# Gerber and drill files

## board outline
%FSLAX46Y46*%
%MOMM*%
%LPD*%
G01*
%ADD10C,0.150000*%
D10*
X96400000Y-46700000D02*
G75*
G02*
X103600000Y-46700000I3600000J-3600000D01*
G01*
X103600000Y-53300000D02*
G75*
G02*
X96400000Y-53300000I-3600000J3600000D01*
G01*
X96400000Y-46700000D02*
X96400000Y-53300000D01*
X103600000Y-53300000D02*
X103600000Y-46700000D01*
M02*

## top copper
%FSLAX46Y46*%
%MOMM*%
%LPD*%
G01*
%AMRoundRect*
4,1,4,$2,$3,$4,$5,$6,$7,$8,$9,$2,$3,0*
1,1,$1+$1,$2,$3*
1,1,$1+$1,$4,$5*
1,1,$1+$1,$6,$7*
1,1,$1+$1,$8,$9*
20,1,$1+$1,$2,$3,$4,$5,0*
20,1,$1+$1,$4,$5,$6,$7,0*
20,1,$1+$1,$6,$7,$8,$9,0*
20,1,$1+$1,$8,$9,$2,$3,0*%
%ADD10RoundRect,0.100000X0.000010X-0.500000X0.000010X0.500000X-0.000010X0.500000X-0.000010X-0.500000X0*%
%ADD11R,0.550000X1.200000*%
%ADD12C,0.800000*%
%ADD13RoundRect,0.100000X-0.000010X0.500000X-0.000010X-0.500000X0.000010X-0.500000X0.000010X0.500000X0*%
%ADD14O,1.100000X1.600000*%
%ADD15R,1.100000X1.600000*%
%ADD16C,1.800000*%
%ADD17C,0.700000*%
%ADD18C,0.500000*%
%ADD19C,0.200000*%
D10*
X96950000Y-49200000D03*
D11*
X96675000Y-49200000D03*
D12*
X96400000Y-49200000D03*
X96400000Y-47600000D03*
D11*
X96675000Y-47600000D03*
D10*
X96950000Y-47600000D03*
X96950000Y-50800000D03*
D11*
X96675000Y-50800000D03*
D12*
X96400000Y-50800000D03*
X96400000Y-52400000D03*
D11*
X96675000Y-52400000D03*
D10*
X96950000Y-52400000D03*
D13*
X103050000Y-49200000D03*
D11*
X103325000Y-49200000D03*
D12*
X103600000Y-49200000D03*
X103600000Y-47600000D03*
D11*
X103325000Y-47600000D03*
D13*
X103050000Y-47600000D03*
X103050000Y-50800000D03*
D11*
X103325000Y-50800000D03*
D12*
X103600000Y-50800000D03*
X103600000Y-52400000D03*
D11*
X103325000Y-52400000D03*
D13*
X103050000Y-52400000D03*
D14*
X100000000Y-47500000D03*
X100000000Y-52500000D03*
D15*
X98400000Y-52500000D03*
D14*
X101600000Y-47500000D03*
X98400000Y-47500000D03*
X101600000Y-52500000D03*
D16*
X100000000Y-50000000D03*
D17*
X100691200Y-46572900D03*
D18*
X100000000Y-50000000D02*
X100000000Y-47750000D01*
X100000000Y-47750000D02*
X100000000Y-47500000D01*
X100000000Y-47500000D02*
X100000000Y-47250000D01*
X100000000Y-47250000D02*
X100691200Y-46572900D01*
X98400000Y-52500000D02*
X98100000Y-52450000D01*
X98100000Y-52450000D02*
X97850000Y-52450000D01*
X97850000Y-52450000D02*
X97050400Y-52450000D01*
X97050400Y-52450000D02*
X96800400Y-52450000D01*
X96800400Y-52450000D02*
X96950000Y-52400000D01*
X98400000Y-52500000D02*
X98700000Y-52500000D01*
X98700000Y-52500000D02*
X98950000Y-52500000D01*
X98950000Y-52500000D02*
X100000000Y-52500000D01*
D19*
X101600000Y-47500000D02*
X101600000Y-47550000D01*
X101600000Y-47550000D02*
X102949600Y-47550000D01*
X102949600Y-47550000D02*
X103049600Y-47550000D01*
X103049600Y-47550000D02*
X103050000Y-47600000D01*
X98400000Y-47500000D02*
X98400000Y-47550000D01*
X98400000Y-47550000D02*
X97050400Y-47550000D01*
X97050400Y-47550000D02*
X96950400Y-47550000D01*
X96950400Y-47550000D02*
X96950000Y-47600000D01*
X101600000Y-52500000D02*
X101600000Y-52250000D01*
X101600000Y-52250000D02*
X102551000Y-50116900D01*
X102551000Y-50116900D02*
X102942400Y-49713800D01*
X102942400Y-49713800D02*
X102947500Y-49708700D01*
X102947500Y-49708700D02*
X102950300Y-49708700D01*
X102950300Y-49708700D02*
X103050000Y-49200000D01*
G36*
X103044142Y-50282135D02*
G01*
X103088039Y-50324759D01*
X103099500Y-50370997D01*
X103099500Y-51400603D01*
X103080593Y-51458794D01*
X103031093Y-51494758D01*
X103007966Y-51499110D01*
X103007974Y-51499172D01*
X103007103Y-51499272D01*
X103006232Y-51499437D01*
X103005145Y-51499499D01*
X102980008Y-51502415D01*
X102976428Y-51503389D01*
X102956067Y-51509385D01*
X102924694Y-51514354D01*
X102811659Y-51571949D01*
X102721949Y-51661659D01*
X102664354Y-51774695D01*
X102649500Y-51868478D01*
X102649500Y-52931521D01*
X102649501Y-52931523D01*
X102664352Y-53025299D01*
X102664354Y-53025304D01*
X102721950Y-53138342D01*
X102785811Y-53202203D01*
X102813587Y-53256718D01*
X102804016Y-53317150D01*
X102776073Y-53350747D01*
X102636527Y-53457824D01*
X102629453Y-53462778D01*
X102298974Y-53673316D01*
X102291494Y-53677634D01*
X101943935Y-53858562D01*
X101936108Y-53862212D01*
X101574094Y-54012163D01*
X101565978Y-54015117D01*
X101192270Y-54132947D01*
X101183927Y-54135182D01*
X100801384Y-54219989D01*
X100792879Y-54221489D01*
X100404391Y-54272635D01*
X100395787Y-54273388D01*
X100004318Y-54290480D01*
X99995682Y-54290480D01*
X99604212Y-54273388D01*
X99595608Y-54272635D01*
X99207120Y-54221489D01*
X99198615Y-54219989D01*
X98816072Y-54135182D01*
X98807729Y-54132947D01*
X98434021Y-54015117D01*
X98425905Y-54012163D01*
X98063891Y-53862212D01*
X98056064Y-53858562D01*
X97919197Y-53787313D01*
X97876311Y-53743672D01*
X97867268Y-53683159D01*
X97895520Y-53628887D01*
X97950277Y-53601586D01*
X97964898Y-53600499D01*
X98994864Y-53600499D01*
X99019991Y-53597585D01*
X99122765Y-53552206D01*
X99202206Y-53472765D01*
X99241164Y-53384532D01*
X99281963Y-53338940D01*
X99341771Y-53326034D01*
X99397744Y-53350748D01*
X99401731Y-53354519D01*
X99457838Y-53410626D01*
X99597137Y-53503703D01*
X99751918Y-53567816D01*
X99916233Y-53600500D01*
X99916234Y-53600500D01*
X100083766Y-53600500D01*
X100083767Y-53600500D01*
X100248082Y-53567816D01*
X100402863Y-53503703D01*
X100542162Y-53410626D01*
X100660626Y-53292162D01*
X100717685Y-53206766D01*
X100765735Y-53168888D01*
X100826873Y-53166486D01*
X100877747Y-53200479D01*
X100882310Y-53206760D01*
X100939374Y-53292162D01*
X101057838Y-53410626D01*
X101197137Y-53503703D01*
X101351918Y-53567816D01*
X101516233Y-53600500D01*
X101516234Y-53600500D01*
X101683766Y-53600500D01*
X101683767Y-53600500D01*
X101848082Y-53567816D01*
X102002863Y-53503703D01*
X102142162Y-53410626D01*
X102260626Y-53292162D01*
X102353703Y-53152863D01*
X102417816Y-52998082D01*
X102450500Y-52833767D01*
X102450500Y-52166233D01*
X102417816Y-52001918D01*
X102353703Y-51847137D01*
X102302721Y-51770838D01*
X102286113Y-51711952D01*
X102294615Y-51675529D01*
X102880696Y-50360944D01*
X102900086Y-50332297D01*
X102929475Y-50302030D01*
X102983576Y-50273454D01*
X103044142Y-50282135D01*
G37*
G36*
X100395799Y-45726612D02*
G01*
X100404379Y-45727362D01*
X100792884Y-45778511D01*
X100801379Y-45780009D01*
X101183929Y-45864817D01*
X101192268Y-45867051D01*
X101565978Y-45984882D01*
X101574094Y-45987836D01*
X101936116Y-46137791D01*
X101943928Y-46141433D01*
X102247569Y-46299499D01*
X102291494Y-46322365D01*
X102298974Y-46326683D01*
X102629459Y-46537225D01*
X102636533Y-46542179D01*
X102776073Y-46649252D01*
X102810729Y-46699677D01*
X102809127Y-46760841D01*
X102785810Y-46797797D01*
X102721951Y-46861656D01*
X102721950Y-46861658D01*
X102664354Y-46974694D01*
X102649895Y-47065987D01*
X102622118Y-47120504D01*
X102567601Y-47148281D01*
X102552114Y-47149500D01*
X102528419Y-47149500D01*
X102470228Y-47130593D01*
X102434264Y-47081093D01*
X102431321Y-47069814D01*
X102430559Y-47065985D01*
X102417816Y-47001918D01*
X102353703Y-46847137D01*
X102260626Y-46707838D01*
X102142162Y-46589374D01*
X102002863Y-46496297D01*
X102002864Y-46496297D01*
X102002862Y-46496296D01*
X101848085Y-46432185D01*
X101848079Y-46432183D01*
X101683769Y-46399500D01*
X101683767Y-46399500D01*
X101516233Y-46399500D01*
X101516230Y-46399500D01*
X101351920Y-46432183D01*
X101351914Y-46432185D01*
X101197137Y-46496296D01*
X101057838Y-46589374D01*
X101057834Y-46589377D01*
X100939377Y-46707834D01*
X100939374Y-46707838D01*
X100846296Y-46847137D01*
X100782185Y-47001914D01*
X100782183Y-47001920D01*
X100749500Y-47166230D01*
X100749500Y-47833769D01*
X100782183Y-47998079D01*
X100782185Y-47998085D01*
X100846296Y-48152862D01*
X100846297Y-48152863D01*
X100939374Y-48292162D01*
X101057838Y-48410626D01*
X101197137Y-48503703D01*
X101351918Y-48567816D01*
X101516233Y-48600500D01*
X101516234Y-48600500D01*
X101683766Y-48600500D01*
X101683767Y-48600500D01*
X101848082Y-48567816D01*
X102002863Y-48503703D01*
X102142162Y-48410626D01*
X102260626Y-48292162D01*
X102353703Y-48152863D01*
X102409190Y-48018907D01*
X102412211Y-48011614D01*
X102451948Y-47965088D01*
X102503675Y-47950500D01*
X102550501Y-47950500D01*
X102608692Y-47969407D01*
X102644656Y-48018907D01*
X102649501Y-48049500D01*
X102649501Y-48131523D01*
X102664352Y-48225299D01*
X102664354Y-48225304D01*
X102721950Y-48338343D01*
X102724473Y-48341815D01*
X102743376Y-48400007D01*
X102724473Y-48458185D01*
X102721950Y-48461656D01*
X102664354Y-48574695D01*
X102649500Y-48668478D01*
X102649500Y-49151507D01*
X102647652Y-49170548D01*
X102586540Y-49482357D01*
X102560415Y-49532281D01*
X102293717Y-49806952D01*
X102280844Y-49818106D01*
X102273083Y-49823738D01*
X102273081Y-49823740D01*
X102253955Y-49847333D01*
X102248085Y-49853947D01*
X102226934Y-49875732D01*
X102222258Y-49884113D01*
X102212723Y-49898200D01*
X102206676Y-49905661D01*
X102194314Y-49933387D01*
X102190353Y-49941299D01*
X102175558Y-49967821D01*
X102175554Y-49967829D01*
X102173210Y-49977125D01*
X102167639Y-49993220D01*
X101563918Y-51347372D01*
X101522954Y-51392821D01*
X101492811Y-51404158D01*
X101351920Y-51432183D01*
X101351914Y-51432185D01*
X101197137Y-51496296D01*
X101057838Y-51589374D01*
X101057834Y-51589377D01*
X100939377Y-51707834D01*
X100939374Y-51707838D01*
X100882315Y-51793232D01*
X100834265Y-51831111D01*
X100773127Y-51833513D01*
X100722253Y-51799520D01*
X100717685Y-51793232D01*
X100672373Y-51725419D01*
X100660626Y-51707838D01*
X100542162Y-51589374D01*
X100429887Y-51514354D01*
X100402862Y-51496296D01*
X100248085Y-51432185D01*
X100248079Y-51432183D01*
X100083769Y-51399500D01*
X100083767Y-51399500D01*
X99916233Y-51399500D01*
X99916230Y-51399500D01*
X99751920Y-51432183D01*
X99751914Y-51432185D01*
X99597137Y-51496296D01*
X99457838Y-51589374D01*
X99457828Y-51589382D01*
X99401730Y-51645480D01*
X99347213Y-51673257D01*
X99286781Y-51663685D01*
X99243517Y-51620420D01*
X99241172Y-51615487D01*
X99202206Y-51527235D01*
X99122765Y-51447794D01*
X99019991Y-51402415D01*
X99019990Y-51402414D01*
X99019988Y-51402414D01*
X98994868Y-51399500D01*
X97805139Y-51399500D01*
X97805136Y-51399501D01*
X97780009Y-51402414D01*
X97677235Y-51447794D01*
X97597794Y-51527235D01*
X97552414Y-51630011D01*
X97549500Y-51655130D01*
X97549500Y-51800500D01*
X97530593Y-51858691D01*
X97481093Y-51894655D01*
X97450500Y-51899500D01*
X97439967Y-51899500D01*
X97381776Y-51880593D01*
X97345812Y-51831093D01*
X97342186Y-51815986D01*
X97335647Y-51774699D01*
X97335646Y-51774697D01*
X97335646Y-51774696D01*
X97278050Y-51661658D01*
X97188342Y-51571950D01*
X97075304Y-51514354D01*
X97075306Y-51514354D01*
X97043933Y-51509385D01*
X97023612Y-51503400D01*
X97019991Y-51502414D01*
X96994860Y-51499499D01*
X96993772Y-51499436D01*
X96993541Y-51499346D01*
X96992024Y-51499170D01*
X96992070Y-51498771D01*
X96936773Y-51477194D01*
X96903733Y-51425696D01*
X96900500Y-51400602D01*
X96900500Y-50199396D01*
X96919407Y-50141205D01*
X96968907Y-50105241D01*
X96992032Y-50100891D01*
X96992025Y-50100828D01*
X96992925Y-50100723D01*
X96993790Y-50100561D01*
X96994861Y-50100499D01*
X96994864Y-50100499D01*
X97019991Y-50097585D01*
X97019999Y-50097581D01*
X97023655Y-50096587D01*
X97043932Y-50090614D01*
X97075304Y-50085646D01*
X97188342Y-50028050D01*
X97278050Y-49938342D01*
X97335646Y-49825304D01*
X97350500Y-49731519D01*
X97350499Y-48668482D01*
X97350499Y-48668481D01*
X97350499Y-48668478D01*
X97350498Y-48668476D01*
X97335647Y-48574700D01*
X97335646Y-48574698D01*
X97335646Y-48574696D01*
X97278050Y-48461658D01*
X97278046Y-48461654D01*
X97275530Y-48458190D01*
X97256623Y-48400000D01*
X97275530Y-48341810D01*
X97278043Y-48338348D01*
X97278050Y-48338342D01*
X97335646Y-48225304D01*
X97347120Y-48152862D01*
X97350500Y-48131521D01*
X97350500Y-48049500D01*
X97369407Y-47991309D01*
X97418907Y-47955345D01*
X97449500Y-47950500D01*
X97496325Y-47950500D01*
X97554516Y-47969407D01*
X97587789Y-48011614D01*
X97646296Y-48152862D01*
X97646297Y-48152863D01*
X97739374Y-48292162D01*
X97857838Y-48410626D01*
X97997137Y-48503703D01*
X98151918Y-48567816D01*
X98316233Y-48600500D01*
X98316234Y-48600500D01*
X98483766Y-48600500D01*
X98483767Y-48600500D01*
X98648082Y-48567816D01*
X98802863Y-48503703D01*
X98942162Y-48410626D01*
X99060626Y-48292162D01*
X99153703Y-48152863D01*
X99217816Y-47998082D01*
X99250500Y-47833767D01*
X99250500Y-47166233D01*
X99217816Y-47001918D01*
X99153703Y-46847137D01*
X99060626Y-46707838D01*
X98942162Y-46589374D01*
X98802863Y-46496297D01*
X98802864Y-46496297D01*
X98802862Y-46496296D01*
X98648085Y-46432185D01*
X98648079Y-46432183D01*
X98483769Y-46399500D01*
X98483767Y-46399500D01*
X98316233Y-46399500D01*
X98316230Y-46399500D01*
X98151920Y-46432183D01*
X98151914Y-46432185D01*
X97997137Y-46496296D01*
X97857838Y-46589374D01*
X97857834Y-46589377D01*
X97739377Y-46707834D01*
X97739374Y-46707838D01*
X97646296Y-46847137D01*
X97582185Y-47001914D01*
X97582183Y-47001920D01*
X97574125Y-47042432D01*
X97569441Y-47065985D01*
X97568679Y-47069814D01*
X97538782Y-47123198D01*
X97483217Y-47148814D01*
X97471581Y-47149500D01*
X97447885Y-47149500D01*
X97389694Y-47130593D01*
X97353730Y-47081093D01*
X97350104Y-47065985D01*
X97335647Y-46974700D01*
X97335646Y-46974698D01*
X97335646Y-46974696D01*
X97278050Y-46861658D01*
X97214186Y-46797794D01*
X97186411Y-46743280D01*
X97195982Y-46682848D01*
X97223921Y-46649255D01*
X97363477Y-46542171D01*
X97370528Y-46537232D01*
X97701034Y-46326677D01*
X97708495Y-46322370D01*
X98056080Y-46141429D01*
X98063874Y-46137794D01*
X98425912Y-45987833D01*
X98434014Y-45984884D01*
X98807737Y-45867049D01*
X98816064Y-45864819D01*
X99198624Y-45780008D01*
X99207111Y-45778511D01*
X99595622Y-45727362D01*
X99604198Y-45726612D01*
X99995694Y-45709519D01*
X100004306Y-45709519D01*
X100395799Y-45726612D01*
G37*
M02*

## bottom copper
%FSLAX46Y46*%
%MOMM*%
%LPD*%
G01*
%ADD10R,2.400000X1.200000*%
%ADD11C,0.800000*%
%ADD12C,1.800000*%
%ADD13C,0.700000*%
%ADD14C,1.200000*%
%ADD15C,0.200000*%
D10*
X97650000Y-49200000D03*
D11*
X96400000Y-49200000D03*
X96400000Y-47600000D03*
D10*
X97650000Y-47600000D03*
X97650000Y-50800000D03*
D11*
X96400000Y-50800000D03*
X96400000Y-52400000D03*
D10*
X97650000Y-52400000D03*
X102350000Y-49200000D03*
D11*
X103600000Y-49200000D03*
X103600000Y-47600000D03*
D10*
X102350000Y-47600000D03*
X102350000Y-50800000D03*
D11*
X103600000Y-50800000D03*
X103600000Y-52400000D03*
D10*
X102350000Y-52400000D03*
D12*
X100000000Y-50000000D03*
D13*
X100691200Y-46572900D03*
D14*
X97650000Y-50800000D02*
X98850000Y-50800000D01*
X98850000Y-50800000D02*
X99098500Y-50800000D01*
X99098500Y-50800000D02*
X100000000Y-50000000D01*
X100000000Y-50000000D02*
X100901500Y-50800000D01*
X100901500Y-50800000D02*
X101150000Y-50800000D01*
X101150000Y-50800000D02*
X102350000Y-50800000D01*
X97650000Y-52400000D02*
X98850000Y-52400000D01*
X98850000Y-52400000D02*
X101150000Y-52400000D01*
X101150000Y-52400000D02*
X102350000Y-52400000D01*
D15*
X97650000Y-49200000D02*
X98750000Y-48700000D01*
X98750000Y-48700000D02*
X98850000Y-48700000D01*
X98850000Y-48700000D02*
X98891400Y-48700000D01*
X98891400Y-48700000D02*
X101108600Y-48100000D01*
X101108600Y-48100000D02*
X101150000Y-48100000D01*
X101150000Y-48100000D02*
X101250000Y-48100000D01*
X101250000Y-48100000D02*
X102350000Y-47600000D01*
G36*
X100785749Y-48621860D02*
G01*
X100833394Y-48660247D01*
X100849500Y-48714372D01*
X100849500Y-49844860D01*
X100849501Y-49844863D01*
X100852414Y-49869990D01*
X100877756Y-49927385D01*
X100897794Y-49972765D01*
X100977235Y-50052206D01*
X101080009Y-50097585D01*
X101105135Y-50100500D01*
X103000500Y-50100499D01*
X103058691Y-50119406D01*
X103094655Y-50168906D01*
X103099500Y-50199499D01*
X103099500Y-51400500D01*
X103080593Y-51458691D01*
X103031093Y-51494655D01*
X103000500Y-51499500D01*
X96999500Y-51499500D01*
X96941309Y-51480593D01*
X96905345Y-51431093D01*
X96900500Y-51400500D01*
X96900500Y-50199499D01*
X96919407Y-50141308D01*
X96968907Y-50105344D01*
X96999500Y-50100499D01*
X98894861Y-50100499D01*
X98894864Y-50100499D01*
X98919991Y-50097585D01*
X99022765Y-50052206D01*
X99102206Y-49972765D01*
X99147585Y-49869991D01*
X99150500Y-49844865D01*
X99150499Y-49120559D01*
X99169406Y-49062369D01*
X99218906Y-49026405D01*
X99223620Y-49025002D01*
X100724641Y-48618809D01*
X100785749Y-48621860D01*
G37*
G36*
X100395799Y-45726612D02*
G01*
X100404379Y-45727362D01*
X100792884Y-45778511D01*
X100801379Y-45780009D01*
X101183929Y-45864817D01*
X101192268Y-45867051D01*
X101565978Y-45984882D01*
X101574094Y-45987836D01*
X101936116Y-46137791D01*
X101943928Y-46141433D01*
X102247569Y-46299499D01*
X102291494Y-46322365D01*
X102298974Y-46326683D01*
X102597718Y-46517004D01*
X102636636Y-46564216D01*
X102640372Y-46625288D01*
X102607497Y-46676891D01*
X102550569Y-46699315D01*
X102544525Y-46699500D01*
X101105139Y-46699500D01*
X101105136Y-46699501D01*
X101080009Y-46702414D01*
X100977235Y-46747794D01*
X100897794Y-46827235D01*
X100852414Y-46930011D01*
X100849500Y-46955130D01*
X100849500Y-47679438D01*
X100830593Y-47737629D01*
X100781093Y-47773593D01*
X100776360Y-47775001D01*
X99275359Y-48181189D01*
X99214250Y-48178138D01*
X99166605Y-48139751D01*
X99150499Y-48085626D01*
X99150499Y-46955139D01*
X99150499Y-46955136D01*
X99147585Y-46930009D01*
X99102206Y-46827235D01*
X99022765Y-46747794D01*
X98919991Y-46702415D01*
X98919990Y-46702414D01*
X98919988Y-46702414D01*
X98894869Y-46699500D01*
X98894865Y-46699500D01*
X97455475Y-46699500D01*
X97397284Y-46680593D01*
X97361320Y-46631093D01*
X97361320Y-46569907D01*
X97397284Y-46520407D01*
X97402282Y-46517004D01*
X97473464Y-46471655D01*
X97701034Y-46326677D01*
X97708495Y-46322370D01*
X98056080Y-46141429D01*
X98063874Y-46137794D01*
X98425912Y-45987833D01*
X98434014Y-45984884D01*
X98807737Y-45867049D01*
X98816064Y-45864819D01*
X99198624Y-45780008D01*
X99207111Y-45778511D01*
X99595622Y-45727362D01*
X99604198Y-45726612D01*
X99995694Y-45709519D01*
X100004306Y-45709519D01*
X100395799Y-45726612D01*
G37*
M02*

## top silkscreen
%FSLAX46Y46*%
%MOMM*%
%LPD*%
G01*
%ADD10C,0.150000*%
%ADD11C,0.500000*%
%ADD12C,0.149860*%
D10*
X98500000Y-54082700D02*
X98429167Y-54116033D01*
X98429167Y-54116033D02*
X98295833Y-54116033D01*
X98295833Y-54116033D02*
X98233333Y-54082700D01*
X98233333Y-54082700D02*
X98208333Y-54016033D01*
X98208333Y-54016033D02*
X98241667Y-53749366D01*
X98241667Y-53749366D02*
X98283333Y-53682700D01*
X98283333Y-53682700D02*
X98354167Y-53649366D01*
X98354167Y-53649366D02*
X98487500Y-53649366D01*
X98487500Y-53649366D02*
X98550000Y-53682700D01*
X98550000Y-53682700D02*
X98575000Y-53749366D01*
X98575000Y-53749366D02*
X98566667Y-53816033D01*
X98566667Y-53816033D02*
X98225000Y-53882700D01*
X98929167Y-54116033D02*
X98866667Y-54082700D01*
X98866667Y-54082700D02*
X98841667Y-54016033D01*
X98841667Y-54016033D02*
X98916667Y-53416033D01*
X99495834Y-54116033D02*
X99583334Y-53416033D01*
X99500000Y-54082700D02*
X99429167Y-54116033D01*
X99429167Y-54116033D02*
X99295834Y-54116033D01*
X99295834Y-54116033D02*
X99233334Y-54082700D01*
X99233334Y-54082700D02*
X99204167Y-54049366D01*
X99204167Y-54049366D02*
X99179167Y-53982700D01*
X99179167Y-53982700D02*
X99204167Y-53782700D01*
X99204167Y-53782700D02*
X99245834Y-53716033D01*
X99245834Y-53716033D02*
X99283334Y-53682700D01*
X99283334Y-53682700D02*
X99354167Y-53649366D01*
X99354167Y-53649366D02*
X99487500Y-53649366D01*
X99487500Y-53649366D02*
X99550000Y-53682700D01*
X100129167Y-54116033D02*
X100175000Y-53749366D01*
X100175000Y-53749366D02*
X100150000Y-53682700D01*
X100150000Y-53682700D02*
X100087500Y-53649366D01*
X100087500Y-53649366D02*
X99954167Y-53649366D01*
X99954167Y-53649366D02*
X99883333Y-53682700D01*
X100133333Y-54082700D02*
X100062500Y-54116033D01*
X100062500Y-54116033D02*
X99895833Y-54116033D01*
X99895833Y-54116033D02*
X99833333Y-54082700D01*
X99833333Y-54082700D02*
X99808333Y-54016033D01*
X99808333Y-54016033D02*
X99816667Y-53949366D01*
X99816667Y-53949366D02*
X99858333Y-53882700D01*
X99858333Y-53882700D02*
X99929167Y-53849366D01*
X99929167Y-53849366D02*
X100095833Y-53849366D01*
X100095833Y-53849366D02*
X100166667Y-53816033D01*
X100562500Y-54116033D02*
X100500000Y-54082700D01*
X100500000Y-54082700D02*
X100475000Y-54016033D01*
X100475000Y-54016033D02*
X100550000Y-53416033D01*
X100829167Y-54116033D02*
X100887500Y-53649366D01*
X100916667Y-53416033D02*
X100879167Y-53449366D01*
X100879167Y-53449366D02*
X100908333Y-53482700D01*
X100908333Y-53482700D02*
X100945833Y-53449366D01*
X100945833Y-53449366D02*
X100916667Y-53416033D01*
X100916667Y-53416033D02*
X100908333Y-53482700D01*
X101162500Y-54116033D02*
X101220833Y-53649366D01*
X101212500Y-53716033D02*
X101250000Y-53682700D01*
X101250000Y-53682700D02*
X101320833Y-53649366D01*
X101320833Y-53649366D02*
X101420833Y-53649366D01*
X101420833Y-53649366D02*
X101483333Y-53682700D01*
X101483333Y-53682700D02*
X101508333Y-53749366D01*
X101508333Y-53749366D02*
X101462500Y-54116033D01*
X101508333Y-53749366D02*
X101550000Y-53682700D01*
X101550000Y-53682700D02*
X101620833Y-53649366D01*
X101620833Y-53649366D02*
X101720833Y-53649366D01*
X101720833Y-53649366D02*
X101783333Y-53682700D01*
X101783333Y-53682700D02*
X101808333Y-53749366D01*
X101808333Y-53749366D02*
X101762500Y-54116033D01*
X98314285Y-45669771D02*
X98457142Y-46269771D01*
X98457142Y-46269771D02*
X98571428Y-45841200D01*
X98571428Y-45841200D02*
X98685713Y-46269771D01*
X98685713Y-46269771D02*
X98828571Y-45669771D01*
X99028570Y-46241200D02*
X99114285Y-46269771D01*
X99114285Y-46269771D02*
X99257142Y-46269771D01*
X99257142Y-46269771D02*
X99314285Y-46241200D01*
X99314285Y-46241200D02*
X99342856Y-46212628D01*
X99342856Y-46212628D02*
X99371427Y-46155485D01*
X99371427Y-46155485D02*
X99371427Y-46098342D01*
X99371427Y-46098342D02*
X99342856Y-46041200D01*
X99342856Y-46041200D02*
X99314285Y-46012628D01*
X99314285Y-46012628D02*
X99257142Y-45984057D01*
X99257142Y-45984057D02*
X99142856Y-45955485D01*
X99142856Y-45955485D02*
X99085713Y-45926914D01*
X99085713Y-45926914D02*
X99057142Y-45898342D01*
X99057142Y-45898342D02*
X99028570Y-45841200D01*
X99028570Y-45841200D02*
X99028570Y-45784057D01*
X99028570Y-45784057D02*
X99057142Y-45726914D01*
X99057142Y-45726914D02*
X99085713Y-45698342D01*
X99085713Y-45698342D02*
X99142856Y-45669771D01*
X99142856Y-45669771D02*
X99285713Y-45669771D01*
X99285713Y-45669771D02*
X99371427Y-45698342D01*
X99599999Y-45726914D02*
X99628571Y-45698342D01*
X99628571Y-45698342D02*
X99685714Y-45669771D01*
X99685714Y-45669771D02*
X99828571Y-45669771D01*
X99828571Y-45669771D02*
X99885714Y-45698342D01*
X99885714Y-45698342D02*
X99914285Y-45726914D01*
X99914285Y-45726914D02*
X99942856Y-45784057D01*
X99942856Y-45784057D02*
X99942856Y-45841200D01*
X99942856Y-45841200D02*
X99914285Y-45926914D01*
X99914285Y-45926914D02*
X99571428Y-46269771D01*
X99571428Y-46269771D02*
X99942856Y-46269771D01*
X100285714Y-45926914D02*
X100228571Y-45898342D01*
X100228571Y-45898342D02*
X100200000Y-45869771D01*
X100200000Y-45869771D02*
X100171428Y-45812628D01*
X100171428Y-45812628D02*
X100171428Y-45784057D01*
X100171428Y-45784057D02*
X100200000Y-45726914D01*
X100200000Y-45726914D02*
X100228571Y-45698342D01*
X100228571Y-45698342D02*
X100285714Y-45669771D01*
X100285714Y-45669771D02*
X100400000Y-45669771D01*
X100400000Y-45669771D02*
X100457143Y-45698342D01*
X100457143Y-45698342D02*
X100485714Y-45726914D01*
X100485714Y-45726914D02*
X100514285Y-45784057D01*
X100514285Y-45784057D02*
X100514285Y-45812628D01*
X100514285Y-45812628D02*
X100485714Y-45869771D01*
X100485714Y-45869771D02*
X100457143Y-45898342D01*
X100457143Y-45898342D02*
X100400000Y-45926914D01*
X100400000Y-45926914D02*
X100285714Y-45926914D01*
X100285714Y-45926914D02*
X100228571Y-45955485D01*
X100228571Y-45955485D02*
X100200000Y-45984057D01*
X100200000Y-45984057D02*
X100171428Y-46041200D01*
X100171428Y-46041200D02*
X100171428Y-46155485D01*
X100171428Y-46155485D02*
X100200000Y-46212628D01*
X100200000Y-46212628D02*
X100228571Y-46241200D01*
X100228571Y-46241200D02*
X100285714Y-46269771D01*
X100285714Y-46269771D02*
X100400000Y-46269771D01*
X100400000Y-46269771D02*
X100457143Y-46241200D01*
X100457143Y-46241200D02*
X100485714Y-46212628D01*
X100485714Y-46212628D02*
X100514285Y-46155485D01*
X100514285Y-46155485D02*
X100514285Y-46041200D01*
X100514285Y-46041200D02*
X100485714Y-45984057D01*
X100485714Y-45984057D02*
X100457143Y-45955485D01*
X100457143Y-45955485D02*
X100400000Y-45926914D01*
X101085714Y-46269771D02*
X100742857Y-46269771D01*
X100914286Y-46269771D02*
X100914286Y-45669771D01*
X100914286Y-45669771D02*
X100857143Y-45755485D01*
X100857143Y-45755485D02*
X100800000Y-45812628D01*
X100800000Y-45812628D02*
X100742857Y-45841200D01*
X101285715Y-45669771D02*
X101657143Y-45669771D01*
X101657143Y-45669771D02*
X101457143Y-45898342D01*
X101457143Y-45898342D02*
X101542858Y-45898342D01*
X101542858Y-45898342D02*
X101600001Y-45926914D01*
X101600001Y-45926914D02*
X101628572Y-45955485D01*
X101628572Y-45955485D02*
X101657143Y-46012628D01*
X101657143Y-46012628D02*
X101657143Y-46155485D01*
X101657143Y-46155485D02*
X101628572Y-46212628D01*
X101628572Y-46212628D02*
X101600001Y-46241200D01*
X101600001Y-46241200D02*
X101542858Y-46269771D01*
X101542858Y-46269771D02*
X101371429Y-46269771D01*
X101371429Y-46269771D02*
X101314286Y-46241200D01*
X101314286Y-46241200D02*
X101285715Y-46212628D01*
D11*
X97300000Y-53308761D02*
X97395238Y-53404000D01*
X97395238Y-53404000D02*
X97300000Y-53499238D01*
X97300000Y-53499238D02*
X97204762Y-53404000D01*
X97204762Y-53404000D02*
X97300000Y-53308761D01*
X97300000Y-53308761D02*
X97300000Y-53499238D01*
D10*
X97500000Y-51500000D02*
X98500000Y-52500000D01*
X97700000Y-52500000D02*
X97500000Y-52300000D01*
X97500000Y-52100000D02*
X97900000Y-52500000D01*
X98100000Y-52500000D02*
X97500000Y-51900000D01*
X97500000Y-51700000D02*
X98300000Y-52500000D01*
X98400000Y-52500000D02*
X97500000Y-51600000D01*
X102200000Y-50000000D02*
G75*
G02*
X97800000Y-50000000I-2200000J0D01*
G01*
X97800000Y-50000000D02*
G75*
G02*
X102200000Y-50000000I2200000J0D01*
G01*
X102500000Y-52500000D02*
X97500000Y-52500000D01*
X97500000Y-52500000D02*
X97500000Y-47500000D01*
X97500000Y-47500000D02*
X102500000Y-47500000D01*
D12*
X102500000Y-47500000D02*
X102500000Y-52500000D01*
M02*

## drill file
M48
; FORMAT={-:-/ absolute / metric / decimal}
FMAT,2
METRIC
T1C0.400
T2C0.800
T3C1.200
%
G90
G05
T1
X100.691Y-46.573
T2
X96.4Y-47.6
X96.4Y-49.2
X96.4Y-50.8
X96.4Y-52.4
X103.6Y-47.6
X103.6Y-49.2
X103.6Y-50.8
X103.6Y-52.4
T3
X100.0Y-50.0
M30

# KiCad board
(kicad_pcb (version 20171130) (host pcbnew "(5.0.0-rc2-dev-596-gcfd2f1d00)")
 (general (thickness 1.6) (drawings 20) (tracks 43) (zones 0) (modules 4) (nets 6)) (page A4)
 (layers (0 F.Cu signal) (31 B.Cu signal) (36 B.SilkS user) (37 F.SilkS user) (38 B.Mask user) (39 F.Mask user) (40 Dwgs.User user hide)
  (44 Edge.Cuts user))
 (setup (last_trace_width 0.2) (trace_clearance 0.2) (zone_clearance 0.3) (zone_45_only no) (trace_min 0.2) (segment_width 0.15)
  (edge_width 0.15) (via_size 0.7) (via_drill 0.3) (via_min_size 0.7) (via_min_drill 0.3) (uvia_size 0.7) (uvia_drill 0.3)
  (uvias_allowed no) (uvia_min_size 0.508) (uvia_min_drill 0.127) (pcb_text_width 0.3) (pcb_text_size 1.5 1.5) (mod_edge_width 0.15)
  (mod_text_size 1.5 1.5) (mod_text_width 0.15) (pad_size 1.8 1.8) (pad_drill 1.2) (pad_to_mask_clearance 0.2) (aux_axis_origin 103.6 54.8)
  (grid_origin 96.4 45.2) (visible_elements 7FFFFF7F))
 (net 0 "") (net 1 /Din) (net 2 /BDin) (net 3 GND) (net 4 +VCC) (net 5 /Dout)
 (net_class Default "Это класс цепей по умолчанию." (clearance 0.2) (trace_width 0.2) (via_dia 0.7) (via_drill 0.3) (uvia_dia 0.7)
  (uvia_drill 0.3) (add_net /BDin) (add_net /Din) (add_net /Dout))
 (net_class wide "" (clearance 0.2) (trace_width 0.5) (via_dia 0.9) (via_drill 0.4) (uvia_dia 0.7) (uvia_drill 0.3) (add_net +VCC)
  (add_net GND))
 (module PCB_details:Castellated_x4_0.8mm (layer F.Cu) (at 96.4 52.4 90)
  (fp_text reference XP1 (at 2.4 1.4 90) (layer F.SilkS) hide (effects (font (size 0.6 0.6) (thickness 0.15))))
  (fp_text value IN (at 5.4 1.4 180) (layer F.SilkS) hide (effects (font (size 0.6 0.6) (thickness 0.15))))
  (pad 3 smd roundrect (at 3.2 0.55 90) (size 1.2 0.2) (layers F.Cu F.Mask) (roundrect_rratio 0.5) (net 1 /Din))
  (pad 3 smd rect (at 3.2 1.25 90) (size 1.2 2.4) (layers B.Cu B.Mask) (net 1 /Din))
  (pad 3 smd rect (at 3.2 0.275 90) (size 1.2 0.55) (layers F.Cu F.Mask) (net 1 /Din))
  (pad 3 thru_hole circle (at 3.2 0 90) (size 0.8 0.8) (drill 0.8) (layers *.Cu) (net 1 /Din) (clearance 0.001))
  (pad 4 thru_hole circle (at 4.8 0 90) (size 0.8 0.8) (drill 0.8) (layers *.Cu) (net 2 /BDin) (clearance 0.001))
  (pad 4 smd rect (at 4.8 0.275 90) (size 1.2 0.55) (layers F.Cu F.Mask) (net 2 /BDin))
  (pad 4 smd rect (at 4.8 1.25 90) (size 1.2 2.4) (layers B.Cu B.Mask) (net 2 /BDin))
  (pad 4 smd roundrect (at 4.8 0.55 90) (size 1.2 0.2) (layers F.Cu F.Mask) (roundrect_rratio 0.5) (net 2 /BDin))
  (pad 2 smd roundrect (at 1.6 0.55 90) (size 1.2 0.2) (layers F.Cu F.Mask) (roundrect_rratio 0.5) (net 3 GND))
  (pad 2 smd rect (at 1.6 1.25 90) (size 1.2 2.4) (layers B.Cu B.Mask) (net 3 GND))
  (pad 2 smd rect (at 1.6 0.275 90) (size 1.2 0.55) (layers F.Cu F.Mask) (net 3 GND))
  (pad 2 thru_hole circle (at 1.6 0 90) (size 0.8 0.8) (drill 0.8) (layers *.Cu) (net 3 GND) (clearance 0.001))
  (pad 1 thru_hole circle (at 0 0 90) (size 0.8 0.8) (drill 0.8) (layers *.Cu) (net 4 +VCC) (clearance 0.001))
  (pad 1 smd rect (at 0 0.275 90) (size 1.2 0.55) (layers F.Cu F.Mask) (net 4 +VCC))
  (pad 1 smd rect (at 0 1.25 90) (size 1.2 2.4) (layers B.Cu B.Mask) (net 4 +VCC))
  (pad 1 smd roundrect (at 0 0.55 90) (size 1.2 0.2) (layers F.Cu F.Mask) (roundrect_rratio 0.5) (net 4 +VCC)))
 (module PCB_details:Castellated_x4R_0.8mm (layer F.Cu) (at 103.6 52.4 270)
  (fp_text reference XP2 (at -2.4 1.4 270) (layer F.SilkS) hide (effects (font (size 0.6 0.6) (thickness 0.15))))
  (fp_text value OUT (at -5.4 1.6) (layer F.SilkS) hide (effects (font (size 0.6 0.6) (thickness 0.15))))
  (pad 3 smd roundrect (at -3.2 0.55 270) (size 1.2 0.2) (layers F.Cu F.Mask) (roundrect_rratio 0.5) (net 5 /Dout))
  (pad 3 smd rect (at -3.2 1.25 270) (size 1.2 2.4) (layers B.Cu B.Mask) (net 5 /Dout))
  (pad 3 smd rect (at -3.2 0.275 270) (size 1.2 0.55) (layers F.Cu F.Mask) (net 5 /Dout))
  (pad 3 thru_hole circle (at -3.2 0 270) (size 0.8 0.8) (drill 0.8) (layers *.Cu) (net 5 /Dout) (clearance 0.001))
  (pad 4 thru_hole circle (at -4.8 0 270) (size 0.8 0.8) (drill 0.8) (layers *.Cu) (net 1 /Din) (clearance 0.001))
  (pad 4 smd rect (at -4.8 0.275 270) (size 1.2 0.55) (layers F.Cu F.Mask) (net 1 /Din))
  (pad 4 smd rect (at -4.8 1.25 270) (size 1.2 2.4) (layers B.Cu B.Mask) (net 1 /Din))
  (pad 4 smd roundrect (at -4.8 0.55 270) (size 1.2 0.2) (layers F.Cu F.Mask) (roundrect_rratio 0.5) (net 1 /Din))
  (pad 2 smd roundrect (at -1.6 0.55 270) (size 1.2 0.2) (layers F.Cu F.Mask) (roundrect_rratio 0.5) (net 3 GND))
  (pad 2 smd rect (at -1.6 1.25 270) (size 1.2 2.4) (layers B.Cu B.Mask) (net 3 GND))
  (pad 2 smd rect (at -1.6 0.275 270) (size 1.2 0.55) (layers F.Cu F.Mask) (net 3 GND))
  (pad 2 thru_hole circle (at -1.6 0 270) (size 0.8 0.8) (drill 0.8) (layers *.Cu) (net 3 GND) (clearance 0.001))
  (pad 1 thru_hole circle (at 0 0 270) (size 0.8 0.8) (drill 0.8) (layers *.Cu) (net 4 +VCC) (clearance 0.001))
  (pad 1 smd rect (at 0 0.275 270) (size 1.2 0.55) (layers F.Cu F.Mask) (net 4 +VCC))
  (pad 1 smd rect (at 0 1.25 270) (size 1.2 2.4) (layers B.Cu B.Mask) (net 4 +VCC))
  (pad 1 smd roundrect (at 0 0.55 270) (size 1.2 0.2) (layers F.Cu F.Mask) (roundrect_rratio 0.5) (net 4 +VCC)))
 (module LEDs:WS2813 (layer F.Cu) (at 100 50 270)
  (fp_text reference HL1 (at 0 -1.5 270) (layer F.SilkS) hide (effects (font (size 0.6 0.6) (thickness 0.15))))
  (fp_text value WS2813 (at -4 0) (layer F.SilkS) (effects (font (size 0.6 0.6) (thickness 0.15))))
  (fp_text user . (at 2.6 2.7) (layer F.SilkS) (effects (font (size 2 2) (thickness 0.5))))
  (fp_line (start 1.5 2.5) (end 2.5 1.5) (layer F.SilkS) (width 0.15))
  (fp_line (start 2.5 2.3) (end 2.3 2.5) (layer F.SilkS) (width 0.15))
  (fp_line (start 2.1 2.5) (end 2.5 2.1) (layer F.SilkS) (width 0.15))
  (fp_line (start 2.5 1.9) (end 1.9 2.5) (layer F.SilkS) (width 0.15))
  (fp_line (start 1.7 2.5) (end 2.5 1.7) (layer F.SilkS) (width 0.15))
  (fp_line (start 2.5 1.6) (end 1.6 2.5) (layer F.SilkS) (width 0.15))
  (fp_circle (center 0 0) (end 0 2.2) (layer F.SilkS) (width 0.15))
  (fp_line (start 2.5 -2.5) (end 2.5 2.5) (layer F.SilkS) (width 0.15))
  (fp_line (start 2.5 2.5) (end -2.5 2.5) (layer F.SilkS) (width 0.15))
  (fp_line (start -2.5 2.5) (end -2.5 -2.5) (layer F.SilkS) (width 0.15))
  (fp_line (start -2.5 -2.5) (end 2.5 -2.5) (layer F.SilkS) (width 0.14986))
  (pad 5 smd oval (at -2.5 0 270) (size 1.6 1.1) (layers F.Cu F.Mask) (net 3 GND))
  (pad 2 smd oval (at 2.5 0 270) (size 1.6 1.1) (layers F.Cu F.Mask) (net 4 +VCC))
  (pad 1 smd rect (at 2.5 1.6 270) (size 1.6 1.1) (layers F.Cu F.Mask) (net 4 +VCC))
  (pad 4 smd oval (at -2.5 -1.6 270) (size 1.6 1.1) (layers F.Cu F.Mask) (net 1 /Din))
  (pad 6 smd oval (at -2.5 1.6 270) (size 1.6 1.1) (layers F.Cu F.Mask) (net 2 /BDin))
  (pad 3 smd oval (at 2.5 -1.6 270) (size 1.6 1.1) (layers F.Cu F.Mask) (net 5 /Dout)))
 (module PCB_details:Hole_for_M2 (layer F.Cu) (at 100 50 270)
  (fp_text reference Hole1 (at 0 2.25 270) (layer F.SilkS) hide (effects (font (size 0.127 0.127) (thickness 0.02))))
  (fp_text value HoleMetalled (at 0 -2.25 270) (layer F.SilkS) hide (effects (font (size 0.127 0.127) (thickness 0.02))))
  (pad H thru_hole circle (at 0 0 270) (size 1.8 1.8) (drill 1.2) (layers *.Cu *.Mask) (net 3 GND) (zone_connect 2)))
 (gr_arc (start 100 50.3) (end 96.4 46.7) (angle 90) (layer Edge.Cuts) (width 0.15))
 (gr_arc (start 100 49.7) (end 103.6 53.3) (angle 90) (layer Edge.Cuts) (width 0.15))
 (gr_line (start 96.4 46.7) (end 96.4 53.3) (angle 90) (layer Edge.Cuts) (width 0.15))
 (gr_line (start 103.6 53.3) (end 103.6 46.7) (angle 90) (layer Edge.Cuts) (width 0.15))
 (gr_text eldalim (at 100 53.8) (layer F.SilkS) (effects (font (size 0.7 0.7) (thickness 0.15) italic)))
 (segment (start 100 50) (end 100 47.75) (width 0.5) (layer F.Cu) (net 3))
 (segment (start 100 47.75) (end 100 47.5) (width 0.5) (layer F.Cu) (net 3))
 (segment (start 100 47.5) (end 100 47.25) (width 0.5) (layer F.Cu) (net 3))
 (segment (start 100 47.25) (end 100.6912 46.5729) (width 0.5) (layer F.Cu) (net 3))
 (segment (start 97.65 50.8) (end 98.85 50.8) (width 1.2) (layer B.Cu) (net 3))
 (segment (start 98.85 50.8) (end 99.0985 50.8) (width 1.2) (layer B.Cu) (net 3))
 (segment (start 99.0985 50.8) (end 100 50) (width 1.2) (layer B.Cu) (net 3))
 (segment (start 100 50) (end 100.9015 50.8) (width 1.2) (layer B.Cu) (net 3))
 (segment (start 100.9015 50.8) (end 101.15 50.8) (width 1.2) (layer B.Cu) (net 3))
 (segment (start 101.15 50.8) (end 102.35 50.8) (width 1.2) (layer B.Cu) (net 3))
 (via (at 100.6912 46.5729) (size 0.7) (layers F.Cu B.Cu) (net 3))
 (segment (start 98.4 52.5) (end 98.1 52.45) (width 0.5) (layer F.Cu) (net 4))
 (segment (start 98.1 52.45) (end 97.85 52.45) (width 0.5) (layer F.Cu) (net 4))
 (segment (start 97.85 52.45) (end 97.0504 52.45) (width 0.5) (layer F.Cu) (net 4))
 (segment (start 97.0504 52.45) (end 96.8004 52.45) (width 0.5) (layer F.Cu) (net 4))
 (segment (start 96.8004 52.45) (end 96.95 52.4) (width 0.5) (layer F.Cu) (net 4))
 (segment (start 98.4 52.5) (end 98.7 52.5) (width 0.5) (layer F.Cu) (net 4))
 (segment (start 98.7 52.5) (end 98.95 52.5) (width 0.5) (layer F.Cu) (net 4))
 (segment (start 98.95 52.5) (end 100 52.5) (width 0.5) (layer F.Cu) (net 4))
 (segment (start 97.65 52.4) (end 98.85 52.4) (width 1.2) (layer B.Cu) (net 4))
 (segment (start 98.85 52.4) (end 101.15 52.4) (width 1.2) (layer B.Cu) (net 4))
 (segment (start 101.15 52.4) (end 102.35 52.4) (width 1.2) (layer B.Cu) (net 4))
 (segment (start 101.6 47.5) (end 101.6 47.55) (width 0.2) (layer F.Cu) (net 1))
 (segment (start 101.6 47.55) (end 102.9496 47.55) (width 0.2) (layer F.Cu) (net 1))
 (segment (start 102.9496 47.55) (end 103.0496 47.55) (width 0.2) (layer F.Cu) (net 1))
 (segment (start 103.0496 47.55) (end 103.05 47.6) (width 0.2) (layer F.Cu) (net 1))
 (segment (start 97.65 49.2) (end 98.75 48.7) (width 0.2) (layer B.Cu) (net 1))
 (segment (start 98.75 48.7) (end 98.85 48.7) (width 0.2) (layer B.Cu) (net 1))
 (segment (start 98.85 48.7) (end 98.8914 48.7) (width 0.2) (layer B.Cu) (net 1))
 (segment (start 98.8914 48.7) (end 101.1086 48.1) (width 0.2) (layer B.Cu) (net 1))
 (segment (start 101.1086 48.1) (end 101.15 48.1) (width 0.2) (layer B.Cu) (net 1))
 (segment (start 101.15 48.1) (end 101.25 48.1) (width 0.2) (layer B.Cu) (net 1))
 (segment (start 101.25 48.1) (end 102.35 47.6) (width 0.2) (layer B.Cu) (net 1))
 (segment (start 98.4 47.5) (end 98.4 47.55) (width 0.2) (layer F.Cu) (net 2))
 (segment (start 98.4 47.55) (end 97.0504 47.55) (width 0.2) (layer F.Cu) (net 2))
 (segment (start 97.0504 47.55) (end 96.9504 47.55) (width 0.2) (layer F.Cu) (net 2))
 (segment (start 96.9504 47.55) (end 96.95 47.6) (width 0.2) (layer F.Cu) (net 2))
 (segment (start 101.6 52.5) (end 101.6 52.25) (width 0.2) (layer F.Cu) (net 5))
 (segment (start 101.6 52.25) (end 102.551 50.1169) (width 0.2) (layer F.Cu) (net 5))
 (segment (start 102.551 50.1169) (end 102.9424 49.7138) (width 0.2) (layer F.Cu) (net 5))
 (segment (start 102.9424 49.7138) (end 102.9475 49.7087) (width 0.2) (layer F.Cu) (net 5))
 (segment (start 102.9475 49.7087) (end 102.9503 49.7087) (width 0.2) (layer F.Cu) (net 5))
 (segment (start 102.9503 49.7087) (end 103.05 49.2) (width 0.2) (layer F.Cu) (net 5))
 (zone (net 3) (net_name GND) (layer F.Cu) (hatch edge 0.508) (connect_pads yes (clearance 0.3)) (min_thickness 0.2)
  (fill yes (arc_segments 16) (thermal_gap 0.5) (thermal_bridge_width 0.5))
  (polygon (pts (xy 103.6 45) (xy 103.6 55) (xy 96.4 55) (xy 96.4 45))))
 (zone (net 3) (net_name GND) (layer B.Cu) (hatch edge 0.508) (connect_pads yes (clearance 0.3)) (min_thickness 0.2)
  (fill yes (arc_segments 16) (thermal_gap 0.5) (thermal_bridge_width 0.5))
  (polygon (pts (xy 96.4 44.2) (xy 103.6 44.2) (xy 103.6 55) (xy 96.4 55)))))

